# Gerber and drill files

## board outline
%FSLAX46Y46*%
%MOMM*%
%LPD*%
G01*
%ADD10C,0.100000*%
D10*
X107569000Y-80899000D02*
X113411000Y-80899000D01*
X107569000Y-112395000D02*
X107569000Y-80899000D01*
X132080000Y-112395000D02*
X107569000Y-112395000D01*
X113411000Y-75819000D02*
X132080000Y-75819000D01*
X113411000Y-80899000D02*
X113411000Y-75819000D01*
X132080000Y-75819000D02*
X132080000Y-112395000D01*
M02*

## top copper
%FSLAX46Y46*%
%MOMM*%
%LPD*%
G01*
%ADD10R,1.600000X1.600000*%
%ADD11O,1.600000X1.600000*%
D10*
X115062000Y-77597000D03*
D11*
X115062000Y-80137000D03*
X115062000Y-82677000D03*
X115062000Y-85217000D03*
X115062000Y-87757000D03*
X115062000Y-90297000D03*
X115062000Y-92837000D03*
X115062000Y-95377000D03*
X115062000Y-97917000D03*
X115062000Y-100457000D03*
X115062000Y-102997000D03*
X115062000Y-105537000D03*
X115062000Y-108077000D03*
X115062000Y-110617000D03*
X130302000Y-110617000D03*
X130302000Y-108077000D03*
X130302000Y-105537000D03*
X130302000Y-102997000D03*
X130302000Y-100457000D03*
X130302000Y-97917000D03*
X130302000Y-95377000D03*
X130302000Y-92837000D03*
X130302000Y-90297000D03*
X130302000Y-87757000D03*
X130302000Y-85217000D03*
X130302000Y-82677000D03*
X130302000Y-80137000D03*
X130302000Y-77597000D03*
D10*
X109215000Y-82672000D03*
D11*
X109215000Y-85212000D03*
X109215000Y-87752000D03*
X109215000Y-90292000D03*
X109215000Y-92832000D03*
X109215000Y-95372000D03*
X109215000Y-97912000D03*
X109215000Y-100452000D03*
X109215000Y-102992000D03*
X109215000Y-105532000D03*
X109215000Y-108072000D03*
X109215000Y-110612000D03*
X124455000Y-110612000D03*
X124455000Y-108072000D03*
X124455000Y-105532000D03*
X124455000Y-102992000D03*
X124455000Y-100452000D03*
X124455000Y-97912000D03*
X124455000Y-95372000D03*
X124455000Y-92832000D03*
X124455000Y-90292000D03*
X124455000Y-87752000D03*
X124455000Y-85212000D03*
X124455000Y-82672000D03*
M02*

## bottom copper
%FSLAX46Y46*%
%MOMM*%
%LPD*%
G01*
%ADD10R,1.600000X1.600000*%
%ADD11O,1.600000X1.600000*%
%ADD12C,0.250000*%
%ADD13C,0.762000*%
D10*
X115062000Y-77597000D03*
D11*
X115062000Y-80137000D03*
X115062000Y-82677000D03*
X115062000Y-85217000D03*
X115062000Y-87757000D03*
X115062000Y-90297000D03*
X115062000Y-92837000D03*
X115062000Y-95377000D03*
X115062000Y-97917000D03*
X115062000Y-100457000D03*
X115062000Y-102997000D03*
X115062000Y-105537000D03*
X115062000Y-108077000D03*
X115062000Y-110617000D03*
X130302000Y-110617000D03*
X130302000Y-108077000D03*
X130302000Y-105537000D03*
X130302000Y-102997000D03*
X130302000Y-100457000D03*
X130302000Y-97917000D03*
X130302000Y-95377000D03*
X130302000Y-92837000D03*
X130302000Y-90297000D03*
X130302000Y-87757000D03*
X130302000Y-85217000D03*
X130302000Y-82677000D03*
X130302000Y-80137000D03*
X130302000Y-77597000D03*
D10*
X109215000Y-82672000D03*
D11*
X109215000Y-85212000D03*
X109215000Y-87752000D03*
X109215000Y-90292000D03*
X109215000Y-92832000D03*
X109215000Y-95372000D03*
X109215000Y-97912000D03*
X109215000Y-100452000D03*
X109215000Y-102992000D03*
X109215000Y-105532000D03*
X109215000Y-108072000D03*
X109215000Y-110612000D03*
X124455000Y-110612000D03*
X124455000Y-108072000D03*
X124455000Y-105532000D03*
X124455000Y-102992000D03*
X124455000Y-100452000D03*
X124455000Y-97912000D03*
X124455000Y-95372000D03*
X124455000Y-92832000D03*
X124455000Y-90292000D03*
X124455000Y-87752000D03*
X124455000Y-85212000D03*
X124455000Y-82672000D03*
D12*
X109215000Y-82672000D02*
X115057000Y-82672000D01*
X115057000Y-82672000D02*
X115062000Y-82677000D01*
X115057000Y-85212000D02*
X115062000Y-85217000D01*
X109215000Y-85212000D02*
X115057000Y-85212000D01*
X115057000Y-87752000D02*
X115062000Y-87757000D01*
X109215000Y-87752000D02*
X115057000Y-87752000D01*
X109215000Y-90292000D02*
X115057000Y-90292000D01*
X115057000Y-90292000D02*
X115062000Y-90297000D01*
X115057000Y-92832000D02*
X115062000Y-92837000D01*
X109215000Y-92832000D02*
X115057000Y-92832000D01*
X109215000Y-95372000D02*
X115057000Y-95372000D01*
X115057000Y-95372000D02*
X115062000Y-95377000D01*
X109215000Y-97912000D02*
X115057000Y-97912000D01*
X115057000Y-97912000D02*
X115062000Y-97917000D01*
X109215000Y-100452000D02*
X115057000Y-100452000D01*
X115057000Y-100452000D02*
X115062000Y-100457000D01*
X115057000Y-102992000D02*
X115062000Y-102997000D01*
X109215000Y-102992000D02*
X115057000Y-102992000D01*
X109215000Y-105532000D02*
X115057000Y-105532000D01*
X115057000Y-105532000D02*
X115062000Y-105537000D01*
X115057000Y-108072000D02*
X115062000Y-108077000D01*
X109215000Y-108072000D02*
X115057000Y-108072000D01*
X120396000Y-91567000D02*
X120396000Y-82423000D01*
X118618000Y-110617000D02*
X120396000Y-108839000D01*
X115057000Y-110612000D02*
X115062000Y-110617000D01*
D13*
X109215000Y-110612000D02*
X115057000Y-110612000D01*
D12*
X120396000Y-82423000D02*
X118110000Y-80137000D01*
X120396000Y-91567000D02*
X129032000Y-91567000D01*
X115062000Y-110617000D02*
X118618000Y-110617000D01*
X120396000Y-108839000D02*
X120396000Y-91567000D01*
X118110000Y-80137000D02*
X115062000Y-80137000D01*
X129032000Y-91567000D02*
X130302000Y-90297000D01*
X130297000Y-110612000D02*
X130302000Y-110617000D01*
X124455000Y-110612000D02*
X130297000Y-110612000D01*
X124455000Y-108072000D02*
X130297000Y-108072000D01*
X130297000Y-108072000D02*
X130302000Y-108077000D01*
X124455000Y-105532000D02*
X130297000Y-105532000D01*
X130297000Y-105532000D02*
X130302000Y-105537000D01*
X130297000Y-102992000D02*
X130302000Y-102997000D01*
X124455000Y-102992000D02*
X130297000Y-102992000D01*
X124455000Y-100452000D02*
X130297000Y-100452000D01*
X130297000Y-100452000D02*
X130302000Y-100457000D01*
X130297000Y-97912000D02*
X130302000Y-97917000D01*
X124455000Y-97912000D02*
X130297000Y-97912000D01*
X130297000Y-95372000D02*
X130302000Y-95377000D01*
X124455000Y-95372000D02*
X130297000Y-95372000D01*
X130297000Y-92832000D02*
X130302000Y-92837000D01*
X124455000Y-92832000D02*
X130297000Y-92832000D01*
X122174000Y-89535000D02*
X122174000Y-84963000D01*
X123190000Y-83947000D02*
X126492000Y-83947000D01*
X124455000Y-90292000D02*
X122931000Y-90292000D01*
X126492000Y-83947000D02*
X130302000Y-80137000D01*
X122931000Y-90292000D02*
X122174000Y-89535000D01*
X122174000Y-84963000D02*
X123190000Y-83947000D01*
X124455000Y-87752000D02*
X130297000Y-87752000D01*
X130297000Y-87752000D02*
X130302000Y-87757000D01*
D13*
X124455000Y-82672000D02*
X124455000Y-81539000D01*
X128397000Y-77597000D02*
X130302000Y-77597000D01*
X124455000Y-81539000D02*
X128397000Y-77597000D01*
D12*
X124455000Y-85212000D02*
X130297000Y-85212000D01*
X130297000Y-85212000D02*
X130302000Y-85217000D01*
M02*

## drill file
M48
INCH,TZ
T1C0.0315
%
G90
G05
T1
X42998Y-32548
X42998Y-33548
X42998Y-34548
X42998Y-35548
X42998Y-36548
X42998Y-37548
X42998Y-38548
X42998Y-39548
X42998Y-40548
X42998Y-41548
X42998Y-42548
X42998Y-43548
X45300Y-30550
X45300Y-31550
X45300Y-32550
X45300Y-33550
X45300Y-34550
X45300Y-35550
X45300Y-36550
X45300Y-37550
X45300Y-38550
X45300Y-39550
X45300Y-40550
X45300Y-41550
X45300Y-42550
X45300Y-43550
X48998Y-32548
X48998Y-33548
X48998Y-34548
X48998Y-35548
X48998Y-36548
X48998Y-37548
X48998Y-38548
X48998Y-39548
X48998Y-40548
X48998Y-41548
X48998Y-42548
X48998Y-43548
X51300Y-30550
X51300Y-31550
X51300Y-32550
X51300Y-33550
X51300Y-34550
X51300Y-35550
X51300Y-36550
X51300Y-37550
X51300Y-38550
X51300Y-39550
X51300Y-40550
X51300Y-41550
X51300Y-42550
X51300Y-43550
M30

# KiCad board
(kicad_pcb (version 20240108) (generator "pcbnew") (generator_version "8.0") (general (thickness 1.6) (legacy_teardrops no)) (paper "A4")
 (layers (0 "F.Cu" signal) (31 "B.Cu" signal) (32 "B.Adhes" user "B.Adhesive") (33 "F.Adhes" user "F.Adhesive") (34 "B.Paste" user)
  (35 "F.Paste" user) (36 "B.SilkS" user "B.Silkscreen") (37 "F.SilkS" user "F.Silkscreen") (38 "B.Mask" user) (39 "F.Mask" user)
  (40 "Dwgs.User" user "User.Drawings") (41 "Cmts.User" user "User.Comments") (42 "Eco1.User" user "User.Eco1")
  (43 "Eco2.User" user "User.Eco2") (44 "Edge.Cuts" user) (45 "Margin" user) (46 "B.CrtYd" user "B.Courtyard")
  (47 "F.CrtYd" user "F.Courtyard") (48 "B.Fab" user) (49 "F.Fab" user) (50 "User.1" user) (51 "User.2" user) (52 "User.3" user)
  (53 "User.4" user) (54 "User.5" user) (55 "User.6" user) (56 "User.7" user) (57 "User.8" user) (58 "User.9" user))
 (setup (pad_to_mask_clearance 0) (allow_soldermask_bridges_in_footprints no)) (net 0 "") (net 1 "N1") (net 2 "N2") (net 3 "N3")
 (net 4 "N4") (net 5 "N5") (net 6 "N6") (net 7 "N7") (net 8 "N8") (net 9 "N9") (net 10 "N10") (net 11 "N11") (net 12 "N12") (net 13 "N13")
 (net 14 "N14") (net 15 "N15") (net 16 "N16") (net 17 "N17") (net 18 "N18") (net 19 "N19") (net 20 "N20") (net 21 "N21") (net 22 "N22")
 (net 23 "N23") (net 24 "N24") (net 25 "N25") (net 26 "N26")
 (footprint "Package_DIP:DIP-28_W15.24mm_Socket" (layer "F.Cu") (at 115.062 77.597)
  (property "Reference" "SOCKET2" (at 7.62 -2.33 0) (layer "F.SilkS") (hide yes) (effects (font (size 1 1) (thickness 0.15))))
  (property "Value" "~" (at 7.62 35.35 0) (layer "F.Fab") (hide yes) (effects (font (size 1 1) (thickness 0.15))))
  (pad "1" thru_hole rect (at 0 0) (size 1.6 1.6) (drill 0.8) (layers "*.Cu" "*.Mask") (remove_unused_layers no) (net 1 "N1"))
  (pad "2" thru_hole oval (at 0 2.54) (size 1.6 1.6) (drill 0.8) (layers "*.Cu" "*.Mask") (remove_unused_layers no) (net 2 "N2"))
  (pad "3" thru_hole oval (at 0 5.08) (size 1.6 1.6) (drill 0.8) (layers "*.Cu" "*.Mask") (remove_unused_layers no) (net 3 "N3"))
  (pad "4" thru_hole oval (at 0 7.62) (size 1.6 1.6) (drill 0.8) (layers "*.Cu" "*.Mask") (remove_unused_layers no) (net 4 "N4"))
  (pad "5" thru_hole oval (at 0 10.16) (size 1.6 1.6) (drill 0.8) (layers "*.Cu" "*.Mask") (remove_unused_layers no) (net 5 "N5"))
  (pad "6" thru_hole oval (at 0 12.7) (size 1.6 1.6) (drill 0.8) (layers "*.Cu" "*.Mask") (remove_unused_layers no) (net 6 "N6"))
  (pad "7" thru_hole oval (at 0 15.24) (size 1.6 1.6) (drill 0.8) (layers "*.Cu" "*.Mask") (remove_unused_layers no) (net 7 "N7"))
  (pad "8" thru_hole oval (at 0 17.78) (size 1.6 1.6) (drill 0.8) (layers "*.Cu" "*.Mask") (remove_unused_layers no) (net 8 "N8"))
  (pad "9" thru_hole oval (at 0 20.32) (size 1.6 1.6) (drill 0.8) (layers "*.Cu" "*.Mask") (remove_unused_layers no) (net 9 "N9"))
  (pad "10" thru_hole oval (at 0 22.86) (size 1.6 1.6) (drill 0.8) (layers "*.Cu" "*.Mask") (remove_unused_layers no) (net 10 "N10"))
  (pad "11" thru_hole oval (at 0 25.4) (size 1.6 1.6) (drill 0.8) (layers "*.Cu" "*.Mask") (remove_unused_layers no) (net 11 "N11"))
  (pad "12" thru_hole oval (at 0 27.94) (size 1.6 1.6) (drill 0.8) (layers "*.Cu" "*.Mask") (remove_unused_layers no) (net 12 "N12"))
  (pad "13" thru_hole oval (at 0 30.48) (size 1.6 1.6) (drill 0.8) (layers "*.Cu" "*.Mask") (remove_unused_layers no) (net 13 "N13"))
  (pad "14" thru_hole oval (at 0 33.02) (size 1.6 1.6) (drill 0.8) (layers "*.Cu" "*.Mask") (remove_unused_layers no) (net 2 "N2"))
  (pad "15" thru_hole oval (at 15.24 33.02) (size 1.6 1.6) (drill 0.8) (layers "*.Cu" "*.Mask") (remove_unused_layers no) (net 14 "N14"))
  (pad "16" thru_hole oval (at 15.24 30.48) (size 1.6 1.6) (drill 0.8) (layers "*.Cu" "*.Mask") (remove_unused_layers no) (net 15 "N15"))
  (pad "17" thru_hole oval (at 15.24 27.94) (size 1.6 1.6) (drill 0.8) (layers "*.Cu" "*.Mask") (remove_unused_layers no) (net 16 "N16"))
  (pad "18" thru_hole oval (at 15.24 25.4) (size 1.6 1.6) (drill 0.8) (layers "*.Cu" "*.Mask") (remove_unused_layers no) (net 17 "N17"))
  (pad "19" thru_hole oval (at 15.24 22.86) (size 1.6 1.6) (drill 0.8) (layers "*.Cu" "*.Mask") (remove_unused_layers no) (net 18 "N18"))
  (pad "20" thru_hole oval (at 15.24 20.32) (size 1.6 1.6) (drill 0.8) (layers "*.Cu" "*.Mask") (remove_unused_layers no) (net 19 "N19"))
  (pad "21" thru_hole oval (at 15.24 17.78) (size 1.6 1.6) (drill 0.8) (layers "*.Cu" "*.Mask") (remove_unused_layers no) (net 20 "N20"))
  (pad "22" thru_hole oval (at 15.24 15.24) (size 1.6 1.6) (drill 0.8) (layers "*.Cu" "*.Mask") (remove_unused_layers no) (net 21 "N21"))
  (pad "23" thru_hole oval (at 15.24 12.7) (size 1.6 1.6) (drill 0.8) (layers "*.Cu" "*.Mask") (remove_unused_layers no) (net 2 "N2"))
  (pad "24" thru_hole oval (at 15.24 10.16) (size 1.6 1.6) (drill 0.8) (layers "*.Cu" "*.Mask") (remove_unused_layers no) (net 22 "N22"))
  (pad "25" thru_hole oval (at 15.24 7.62) (size 1.6 1.6) (drill 0.8) (layers "*.Cu" "*.Mask") (remove_unused_layers no) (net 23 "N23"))
  (pad "26" thru_hole oval (at 15.24 5.08) (size 1.6 1.6) (drill 0.8) (layers "*.Cu" "*.Mask") (remove_unused_layers no) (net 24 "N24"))
  (pad "27" thru_hole oval (at 15.24 2.54) (size 1.6 1.6) (drill 0.8) (layers "*.Cu" "*.Mask") (remove_unused_layers no) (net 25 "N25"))
  (pad "28" thru_hole oval (at 15.24 0) (size 1.6 1.6) (drill 0.8) (layers "*.Cu" "*.Mask") (remove_unused_layers no) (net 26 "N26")))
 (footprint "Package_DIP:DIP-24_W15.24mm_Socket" (layer "F.Cu") (at 109.215 82.672)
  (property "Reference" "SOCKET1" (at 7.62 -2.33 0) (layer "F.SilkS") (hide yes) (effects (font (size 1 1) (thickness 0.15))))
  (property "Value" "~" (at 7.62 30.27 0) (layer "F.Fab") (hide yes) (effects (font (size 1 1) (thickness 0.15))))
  (pad "1" thru_hole rect (at 0 0) (size 1.6 1.6) (drill 0.8) (layers "*.Cu" "*.Mask") (remove_unused_layers no) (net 3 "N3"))
  (pad "2" thru_hole oval (at 0 2.54) (size 1.6 1.6) (drill 0.8) (layers "*.Cu" "*.Mask") (remove_unused_layers no) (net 4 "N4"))
  (pad "3" thru_hole oval (at 0 5.08) (size 1.6 1.6) (drill 0.8) (layers "*.Cu" "*.Mask") (remove_unused_layers no) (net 5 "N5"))
  (pad "4" thru_hole oval (at 0 7.62) (size 1.6 1.6) (drill 0.8) (layers "*.Cu" "*.Mask") (remove_unused_layers no) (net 6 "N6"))
  (pad "5" thru_hole oval (at 0 10.16) (size 1.6 1.6) (drill 0.8) (layers "*.Cu" "*.Mask") (remove_unused_layers no) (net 7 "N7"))
  (pad "6" thru_hole oval (at 0 12.7) (size 1.6 1.6) (drill 0.8) (layers "*.Cu" "*.Mask") (remove_unused_layers no) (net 8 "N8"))
  (pad "7" thru_hole oval (at 0 15.24) (size 1.6 1.6) (drill 0.8) (layers "*.Cu" "*.Mask") (remove_unused_layers no) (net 9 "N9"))
  (pad "8" thru_hole oval (at 0 17.78) (size 1.6 1.6) (drill 0.8) (layers "*.Cu" "*.Mask") (remove_unused_layers no) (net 10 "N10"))
  (pad "9" thru_hole oval (at 0 20.32) (size 1.6 1.6) (drill 0.8) (layers "*.Cu" "*.Mask") (remove_unused_layers no) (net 11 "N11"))
  (pad "10" thru_hole oval (at 0 22.86) (size 1.6 1.6) (drill 0.8) (layers "*.Cu" "*.Mask") (remove_unused_layers no) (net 12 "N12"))
  (pad "11" thru_hole oval (at 0 25.4) (size 1.6 1.6) (drill 0.8) (layers "*.Cu" "*.Mask") (remove_unused_layers no) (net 13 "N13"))
  (pad "12" thru_hole oval (at 0 27.94) (size 1.6 1.6) (drill 0.8) (layers "*.Cu" "*.Mask") (remove_unused_layers no) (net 2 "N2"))
  (pad "13" thru_hole oval (at 15.24 27.94) (size 1.6 1.6) (drill 0.8) (layers "*.Cu" "*.Mask") (remove_unused_layers no) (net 14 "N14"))
  (pad "14" thru_hole oval (at 15.24 25.4) (size 1.6 1.6) (drill 0.8) (layers "*.Cu" "*.Mask") (remove_unused_layers no) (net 15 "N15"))
  (pad "15" thru_hole oval (at 15.24 22.86) (size 1.6 1.6) (drill 0.8) (layers "*.Cu" "*.Mask") (remove_unused_layers no) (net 16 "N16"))
  (pad "16" thru_hole oval (at 15.24 20.32) (size 1.6 1.6) (drill 0.8) (layers "*.Cu" "*.Mask") (remove_unused_layers no) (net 17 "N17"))
  (pad "17" thru_hole oval (at 15.24 17.78) (size 1.6 1.6) (drill 0.8) (layers "*.Cu" "*.Mask") (remove_unused_layers no) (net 18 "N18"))
  (pad "18" thru_hole oval (at 15.24 15.24) (size 1.6 1.6) (drill 0.8) (layers "*.Cu" "*.Mask") (remove_unused_layers no) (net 19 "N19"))
  (pad "19" thru_hole oval (at 15.24 12.7) (size 1.6 1.6) (drill 0.8) (layers "*.Cu" "*.Mask") (remove_unused_layers no) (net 20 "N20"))
  (pad "20" thru_hole oval (at 15.24 10.16) (size 1.6 1.6) (drill 0.8) (layers "*.Cu" "*.Mask") (remove_unused_layers no) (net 21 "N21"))
  (pad "21" thru_hole oval (at 15.24 7.62) (size 1.6 1.6) (drill 0.8) (layers "*.Cu" "*.Mask") (remove_unused_layers no) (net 25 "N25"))
  (pad "22" thru_hole oval (at 15.24 5.08) (size 1.6 1.6) (drill 0.8) (layers "*.Cu" "*.Mask") (remove_unused_layers no) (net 22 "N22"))
  (pad "23" thru_hole oval (at 15.24 2.54) (size 1.6 1.6) (drill 0.8) (layers "*.Cu" "*.Mask") (remove_unused_layers no) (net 23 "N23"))
  (pad "24" thru_hole oval (at 15.24 0) (size 1.6 1.6) (drill 0.8) (layers "*.Cu" "*.Mask") (remove_unused_layers no) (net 26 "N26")))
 (gr_line (start 107.569 80.899) (end 113.411 80.899) (stroke (width 0.1) (type default)) (layer "Edge.Cuts"))
 (gr_line (start 107.569 112.395) (end 107.569 80.899) (stroke (width 0.1) (type default)) (layer "Edge.Cuts"))
 (gr_line (start 132.08 112.395) (end 107.569 112.395) (stroke (width 0.1) (type default)) (layer "Edge.Cuts"))
 (gr_line (start 113.411 75.819) (end 132.08 75.819) (stroke (width 0.1) (type default)) (layer "Edge.Cuts"))
 (gr_line (start 113.411 80.899) (end 113.411 75.819) (stroke (width 0.1) (type default)) (layer "Edge.Cuts"))
 (gr_line (start 132.08 75.819) (end 132.08 112.395) (stroke (width 0.1) (type default)) (layer "Edge.Cuts"))
 (segment (start 109.215 82.672) (end 115.057 82.672) (width 0.25) (layer "B.Cu") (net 3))
 (segment (start 115.057 82.672) (end 115.062 82.677) (width 0.25) (layer "B.Cu") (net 3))
 (segment (start 115.057 85.212) (end 115.062 85.217) (width 0.25) (layer "B.Cu") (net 4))
 (segment (start 109.215 85.212) (end 115.057 85.212) (width 0.25) (layer "B.Cu") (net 4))
 (segment (start 115.057 87.752) (end 115.062 87.757) (width 0.25) (layer "B.Cu") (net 5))
 (segment (start 109.215 87.752) (end 115.057 87.752) (width 0.25) (layer "B.Cu") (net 5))
 (segment (start 109.215 90.292) (end 115.057 90.292) (width 0.25) (layer "B.Cu") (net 6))
 (segment (start 115.057 90.292) (end 115.062 90.297) (width 0.25) (layer "B.Cu") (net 6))
 (segment (start 115.057 92.832) (end 115.062 92.837) (width 0.25) (layer "B.Cu") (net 7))
 (segment (start 109.215 92.832) (end 115.057 92.832) (width 0.25) (layer "B.Cu") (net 7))
 (segment (start 109.215 95.372) (end 115.057 95.372) (width 0.25) (layer "B.Cu") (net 8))
 (segment (start 115.057 95.372) (end 115.062 95.377) (width 0.25) (layer "B.Cu") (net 8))
 (segment (start 109.215 97.912) (end 115.057 97.912) (width 0.25) (layer "B.Cu") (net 9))
 (segment (start 115.057 97.912) (end 115.062 97.917) (width 0.25) (layer "B.Cu") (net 9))
 (segment (start 109.215 100.452) (end 115.057 100.452) (width 0.25) (layer "B.Cu") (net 10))
 (segment (start 115.057 100.452) (end 115.062 100.457) (width 0.25) (layer "B.Cu") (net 10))
 (segment (start 115.057 102.992) (end 115.062 102.997) (width 0.25) (layer "B.Cu") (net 11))
 (segment (start 109.215 102.992) (end 115.057 102.992) (width 0.25) (layer "B.Cu") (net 11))
 (segment (start 109.215 105.532) (end 115.057 105.532) (width 0.25) (layer "B.Cu") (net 12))
 (segment (start 115.057 105.532) (end 115.062 105.537) (width 0.25) (layer "B.Cu") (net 12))
 (segment (start 115.057 108.072) (end 115.062 108.077) (width 0.25) (layer "B.Cu") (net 13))
 (segment (start 109.215 108.072) (end 115.057 108.072) (width 0.25) (layer "B.Cu") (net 13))
 (segment (start 120.396 91.567) (end 120.396 82.423) (width 0.25) (layer "B.Cu") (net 2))
 (segment (start 118.618 110.617) (end 120.396 108.839) (width 0.25) (layer "B.Cu") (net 2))
 (segment (start 115.057 110.612) (end 115.062 110.617) (width 0.25) (layer "B.Cu") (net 2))
 (segment (start 109.215 110.612) (end 115.057 110.612) (width 0.762) (layer "B.Cu") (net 2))
 (segment (start 120.396 82.423) (end 118.11 80.137) (width 0.25) (layer "B.Cu") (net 2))
 (segment (start 120.396 91.567) (end 129.032 91.567) (width 0.25) (layer "B.Cu") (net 2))
 (segment (start 115.062 110.617) (end 118.618 110.617) (width 0.25) (layer "B.Cu") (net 2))
 (segment (start 120.396 108.839) (end 120.396 91.567) (width 0.25) (layer "B.Cu") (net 2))
 (segment (start 118.11 80.137) (end 115.062 80.137) (width 0.25) (layer "B.Cu") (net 2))
 (segment (start 129.032 91.567) (end 130.302 90.297) (width 0.25) (layer "B.Cu") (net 2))
 (segment (start 130.297 110.612) (end 130.302 110.617) (width 0.25) (layer "B.Cu") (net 14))
 (segment (start 124.455 110.612) (end 130.297 110.612) (width 0.25) (layer "B.Cu") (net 14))
 (segment (start 124.455 108.072) (end 130.297 108.072) (width 0.25) (layer "B.Cu") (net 15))
 (segment (start 130.297 108.072) (end 130.302 108.077) (width 0.25) (layer "B.Cu") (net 15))
 (segment (start 124.455 105.532) (end 130.297 105.532) (width 0.25) (layer "B.Cu") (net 16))
 (segment (start 130.297 105.532) (end 130.302 105.537) (width 0.25) (layer "B.Cu") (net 16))
 (segment (start 130.297 102.992) (end 130.302 102.997) (width 0.25) (layer "B.Cu") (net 17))
 (segment (start 124.455 102.992) (end 130.297 102.992) (width 0.25) (layer "B.Cu") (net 17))
 (segment (start 124.455 100.452) (end 130.297 100.452) (width 0.25) (layer "B.Cu") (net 18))
 (segment (start 130.297 100.452) (end 130.302 100.457) (width 0.25) (layer "B.Cu") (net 18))
 (segment (start 130.297 97.912) (end 130.302 97.917) (width 0.25) (layer "B.Cu") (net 19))
 (segment (start 124.455 97.912) (end 130.297 97.912) (width 0.25) (layer "B.Cu") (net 19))
 (segment (start 130.297 95.372) (end 130.302 95.377) (width 0.25) (layer "B.Cu") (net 20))
 (segment (start 124.455 95.372) (end 130.297 95.372) (width 0.25) (layer "B.Cu") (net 20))
 (segment (start 130.297 92.832) (end 130.302 92.837) (width 0.25) (layer "B.Cu") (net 21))
 (segment (start 124.455 92.832) (end 130.297 92.832) (width 0.25) (layer "B.Cu") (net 21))
 (segment (start 122.174 89.535) (end 122.174 84.963) (width 0.25) (layer "B.Cu") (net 25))
 (segment (start 123.19 83.947) (end 126.492 83.947) (width 0.25) (layer "B.Cu") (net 25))
 (segment (start 124.455 90.292) (end 122.931 90.292) (width 0.25) (layer "B.Cu") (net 25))
 (segment (start 126.492 83.947) (end 130.302 80.137) (width 0.25) (layer "B.Cu") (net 25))
 (segment (start 122.931 90.292) (end 122.174 89.535) (width 0.25) (layer "B.Cu") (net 25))
 (segment (start 122.174 84.963) (end 123.19 83.947) (width 0.25) (layer "B.Cu") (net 25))
 (segment (start 124.455 87.752) (end 130.297 87.752) (width 0.25) (layer "B.Cu") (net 22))
 (segment (start 130.297 87.752) (end 130.302 87.757) (width 0.25) (layer "B.Cu") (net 22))
 (segment (start 124.455 82.672) (end 124.455 81.539) (width 0.762) (layer "B.Cu") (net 26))
 (segment (start 128.397 77.597) (end 130.302 77.597) (width 0.762) (layer "B.Cu") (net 26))
 (segment (start 124.455 81.539) (end 128.397 77.597) (width 0.762) (layer "B.Cu") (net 26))
 (segment (start 124.455 85.212) (end 130.297 85.212) (width 0.25) (layer "B.Cu") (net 23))
 (segment (start 130.297 85.212) (end 130.302 85.217) (width 0.25) (layer "B.Cu") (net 23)))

